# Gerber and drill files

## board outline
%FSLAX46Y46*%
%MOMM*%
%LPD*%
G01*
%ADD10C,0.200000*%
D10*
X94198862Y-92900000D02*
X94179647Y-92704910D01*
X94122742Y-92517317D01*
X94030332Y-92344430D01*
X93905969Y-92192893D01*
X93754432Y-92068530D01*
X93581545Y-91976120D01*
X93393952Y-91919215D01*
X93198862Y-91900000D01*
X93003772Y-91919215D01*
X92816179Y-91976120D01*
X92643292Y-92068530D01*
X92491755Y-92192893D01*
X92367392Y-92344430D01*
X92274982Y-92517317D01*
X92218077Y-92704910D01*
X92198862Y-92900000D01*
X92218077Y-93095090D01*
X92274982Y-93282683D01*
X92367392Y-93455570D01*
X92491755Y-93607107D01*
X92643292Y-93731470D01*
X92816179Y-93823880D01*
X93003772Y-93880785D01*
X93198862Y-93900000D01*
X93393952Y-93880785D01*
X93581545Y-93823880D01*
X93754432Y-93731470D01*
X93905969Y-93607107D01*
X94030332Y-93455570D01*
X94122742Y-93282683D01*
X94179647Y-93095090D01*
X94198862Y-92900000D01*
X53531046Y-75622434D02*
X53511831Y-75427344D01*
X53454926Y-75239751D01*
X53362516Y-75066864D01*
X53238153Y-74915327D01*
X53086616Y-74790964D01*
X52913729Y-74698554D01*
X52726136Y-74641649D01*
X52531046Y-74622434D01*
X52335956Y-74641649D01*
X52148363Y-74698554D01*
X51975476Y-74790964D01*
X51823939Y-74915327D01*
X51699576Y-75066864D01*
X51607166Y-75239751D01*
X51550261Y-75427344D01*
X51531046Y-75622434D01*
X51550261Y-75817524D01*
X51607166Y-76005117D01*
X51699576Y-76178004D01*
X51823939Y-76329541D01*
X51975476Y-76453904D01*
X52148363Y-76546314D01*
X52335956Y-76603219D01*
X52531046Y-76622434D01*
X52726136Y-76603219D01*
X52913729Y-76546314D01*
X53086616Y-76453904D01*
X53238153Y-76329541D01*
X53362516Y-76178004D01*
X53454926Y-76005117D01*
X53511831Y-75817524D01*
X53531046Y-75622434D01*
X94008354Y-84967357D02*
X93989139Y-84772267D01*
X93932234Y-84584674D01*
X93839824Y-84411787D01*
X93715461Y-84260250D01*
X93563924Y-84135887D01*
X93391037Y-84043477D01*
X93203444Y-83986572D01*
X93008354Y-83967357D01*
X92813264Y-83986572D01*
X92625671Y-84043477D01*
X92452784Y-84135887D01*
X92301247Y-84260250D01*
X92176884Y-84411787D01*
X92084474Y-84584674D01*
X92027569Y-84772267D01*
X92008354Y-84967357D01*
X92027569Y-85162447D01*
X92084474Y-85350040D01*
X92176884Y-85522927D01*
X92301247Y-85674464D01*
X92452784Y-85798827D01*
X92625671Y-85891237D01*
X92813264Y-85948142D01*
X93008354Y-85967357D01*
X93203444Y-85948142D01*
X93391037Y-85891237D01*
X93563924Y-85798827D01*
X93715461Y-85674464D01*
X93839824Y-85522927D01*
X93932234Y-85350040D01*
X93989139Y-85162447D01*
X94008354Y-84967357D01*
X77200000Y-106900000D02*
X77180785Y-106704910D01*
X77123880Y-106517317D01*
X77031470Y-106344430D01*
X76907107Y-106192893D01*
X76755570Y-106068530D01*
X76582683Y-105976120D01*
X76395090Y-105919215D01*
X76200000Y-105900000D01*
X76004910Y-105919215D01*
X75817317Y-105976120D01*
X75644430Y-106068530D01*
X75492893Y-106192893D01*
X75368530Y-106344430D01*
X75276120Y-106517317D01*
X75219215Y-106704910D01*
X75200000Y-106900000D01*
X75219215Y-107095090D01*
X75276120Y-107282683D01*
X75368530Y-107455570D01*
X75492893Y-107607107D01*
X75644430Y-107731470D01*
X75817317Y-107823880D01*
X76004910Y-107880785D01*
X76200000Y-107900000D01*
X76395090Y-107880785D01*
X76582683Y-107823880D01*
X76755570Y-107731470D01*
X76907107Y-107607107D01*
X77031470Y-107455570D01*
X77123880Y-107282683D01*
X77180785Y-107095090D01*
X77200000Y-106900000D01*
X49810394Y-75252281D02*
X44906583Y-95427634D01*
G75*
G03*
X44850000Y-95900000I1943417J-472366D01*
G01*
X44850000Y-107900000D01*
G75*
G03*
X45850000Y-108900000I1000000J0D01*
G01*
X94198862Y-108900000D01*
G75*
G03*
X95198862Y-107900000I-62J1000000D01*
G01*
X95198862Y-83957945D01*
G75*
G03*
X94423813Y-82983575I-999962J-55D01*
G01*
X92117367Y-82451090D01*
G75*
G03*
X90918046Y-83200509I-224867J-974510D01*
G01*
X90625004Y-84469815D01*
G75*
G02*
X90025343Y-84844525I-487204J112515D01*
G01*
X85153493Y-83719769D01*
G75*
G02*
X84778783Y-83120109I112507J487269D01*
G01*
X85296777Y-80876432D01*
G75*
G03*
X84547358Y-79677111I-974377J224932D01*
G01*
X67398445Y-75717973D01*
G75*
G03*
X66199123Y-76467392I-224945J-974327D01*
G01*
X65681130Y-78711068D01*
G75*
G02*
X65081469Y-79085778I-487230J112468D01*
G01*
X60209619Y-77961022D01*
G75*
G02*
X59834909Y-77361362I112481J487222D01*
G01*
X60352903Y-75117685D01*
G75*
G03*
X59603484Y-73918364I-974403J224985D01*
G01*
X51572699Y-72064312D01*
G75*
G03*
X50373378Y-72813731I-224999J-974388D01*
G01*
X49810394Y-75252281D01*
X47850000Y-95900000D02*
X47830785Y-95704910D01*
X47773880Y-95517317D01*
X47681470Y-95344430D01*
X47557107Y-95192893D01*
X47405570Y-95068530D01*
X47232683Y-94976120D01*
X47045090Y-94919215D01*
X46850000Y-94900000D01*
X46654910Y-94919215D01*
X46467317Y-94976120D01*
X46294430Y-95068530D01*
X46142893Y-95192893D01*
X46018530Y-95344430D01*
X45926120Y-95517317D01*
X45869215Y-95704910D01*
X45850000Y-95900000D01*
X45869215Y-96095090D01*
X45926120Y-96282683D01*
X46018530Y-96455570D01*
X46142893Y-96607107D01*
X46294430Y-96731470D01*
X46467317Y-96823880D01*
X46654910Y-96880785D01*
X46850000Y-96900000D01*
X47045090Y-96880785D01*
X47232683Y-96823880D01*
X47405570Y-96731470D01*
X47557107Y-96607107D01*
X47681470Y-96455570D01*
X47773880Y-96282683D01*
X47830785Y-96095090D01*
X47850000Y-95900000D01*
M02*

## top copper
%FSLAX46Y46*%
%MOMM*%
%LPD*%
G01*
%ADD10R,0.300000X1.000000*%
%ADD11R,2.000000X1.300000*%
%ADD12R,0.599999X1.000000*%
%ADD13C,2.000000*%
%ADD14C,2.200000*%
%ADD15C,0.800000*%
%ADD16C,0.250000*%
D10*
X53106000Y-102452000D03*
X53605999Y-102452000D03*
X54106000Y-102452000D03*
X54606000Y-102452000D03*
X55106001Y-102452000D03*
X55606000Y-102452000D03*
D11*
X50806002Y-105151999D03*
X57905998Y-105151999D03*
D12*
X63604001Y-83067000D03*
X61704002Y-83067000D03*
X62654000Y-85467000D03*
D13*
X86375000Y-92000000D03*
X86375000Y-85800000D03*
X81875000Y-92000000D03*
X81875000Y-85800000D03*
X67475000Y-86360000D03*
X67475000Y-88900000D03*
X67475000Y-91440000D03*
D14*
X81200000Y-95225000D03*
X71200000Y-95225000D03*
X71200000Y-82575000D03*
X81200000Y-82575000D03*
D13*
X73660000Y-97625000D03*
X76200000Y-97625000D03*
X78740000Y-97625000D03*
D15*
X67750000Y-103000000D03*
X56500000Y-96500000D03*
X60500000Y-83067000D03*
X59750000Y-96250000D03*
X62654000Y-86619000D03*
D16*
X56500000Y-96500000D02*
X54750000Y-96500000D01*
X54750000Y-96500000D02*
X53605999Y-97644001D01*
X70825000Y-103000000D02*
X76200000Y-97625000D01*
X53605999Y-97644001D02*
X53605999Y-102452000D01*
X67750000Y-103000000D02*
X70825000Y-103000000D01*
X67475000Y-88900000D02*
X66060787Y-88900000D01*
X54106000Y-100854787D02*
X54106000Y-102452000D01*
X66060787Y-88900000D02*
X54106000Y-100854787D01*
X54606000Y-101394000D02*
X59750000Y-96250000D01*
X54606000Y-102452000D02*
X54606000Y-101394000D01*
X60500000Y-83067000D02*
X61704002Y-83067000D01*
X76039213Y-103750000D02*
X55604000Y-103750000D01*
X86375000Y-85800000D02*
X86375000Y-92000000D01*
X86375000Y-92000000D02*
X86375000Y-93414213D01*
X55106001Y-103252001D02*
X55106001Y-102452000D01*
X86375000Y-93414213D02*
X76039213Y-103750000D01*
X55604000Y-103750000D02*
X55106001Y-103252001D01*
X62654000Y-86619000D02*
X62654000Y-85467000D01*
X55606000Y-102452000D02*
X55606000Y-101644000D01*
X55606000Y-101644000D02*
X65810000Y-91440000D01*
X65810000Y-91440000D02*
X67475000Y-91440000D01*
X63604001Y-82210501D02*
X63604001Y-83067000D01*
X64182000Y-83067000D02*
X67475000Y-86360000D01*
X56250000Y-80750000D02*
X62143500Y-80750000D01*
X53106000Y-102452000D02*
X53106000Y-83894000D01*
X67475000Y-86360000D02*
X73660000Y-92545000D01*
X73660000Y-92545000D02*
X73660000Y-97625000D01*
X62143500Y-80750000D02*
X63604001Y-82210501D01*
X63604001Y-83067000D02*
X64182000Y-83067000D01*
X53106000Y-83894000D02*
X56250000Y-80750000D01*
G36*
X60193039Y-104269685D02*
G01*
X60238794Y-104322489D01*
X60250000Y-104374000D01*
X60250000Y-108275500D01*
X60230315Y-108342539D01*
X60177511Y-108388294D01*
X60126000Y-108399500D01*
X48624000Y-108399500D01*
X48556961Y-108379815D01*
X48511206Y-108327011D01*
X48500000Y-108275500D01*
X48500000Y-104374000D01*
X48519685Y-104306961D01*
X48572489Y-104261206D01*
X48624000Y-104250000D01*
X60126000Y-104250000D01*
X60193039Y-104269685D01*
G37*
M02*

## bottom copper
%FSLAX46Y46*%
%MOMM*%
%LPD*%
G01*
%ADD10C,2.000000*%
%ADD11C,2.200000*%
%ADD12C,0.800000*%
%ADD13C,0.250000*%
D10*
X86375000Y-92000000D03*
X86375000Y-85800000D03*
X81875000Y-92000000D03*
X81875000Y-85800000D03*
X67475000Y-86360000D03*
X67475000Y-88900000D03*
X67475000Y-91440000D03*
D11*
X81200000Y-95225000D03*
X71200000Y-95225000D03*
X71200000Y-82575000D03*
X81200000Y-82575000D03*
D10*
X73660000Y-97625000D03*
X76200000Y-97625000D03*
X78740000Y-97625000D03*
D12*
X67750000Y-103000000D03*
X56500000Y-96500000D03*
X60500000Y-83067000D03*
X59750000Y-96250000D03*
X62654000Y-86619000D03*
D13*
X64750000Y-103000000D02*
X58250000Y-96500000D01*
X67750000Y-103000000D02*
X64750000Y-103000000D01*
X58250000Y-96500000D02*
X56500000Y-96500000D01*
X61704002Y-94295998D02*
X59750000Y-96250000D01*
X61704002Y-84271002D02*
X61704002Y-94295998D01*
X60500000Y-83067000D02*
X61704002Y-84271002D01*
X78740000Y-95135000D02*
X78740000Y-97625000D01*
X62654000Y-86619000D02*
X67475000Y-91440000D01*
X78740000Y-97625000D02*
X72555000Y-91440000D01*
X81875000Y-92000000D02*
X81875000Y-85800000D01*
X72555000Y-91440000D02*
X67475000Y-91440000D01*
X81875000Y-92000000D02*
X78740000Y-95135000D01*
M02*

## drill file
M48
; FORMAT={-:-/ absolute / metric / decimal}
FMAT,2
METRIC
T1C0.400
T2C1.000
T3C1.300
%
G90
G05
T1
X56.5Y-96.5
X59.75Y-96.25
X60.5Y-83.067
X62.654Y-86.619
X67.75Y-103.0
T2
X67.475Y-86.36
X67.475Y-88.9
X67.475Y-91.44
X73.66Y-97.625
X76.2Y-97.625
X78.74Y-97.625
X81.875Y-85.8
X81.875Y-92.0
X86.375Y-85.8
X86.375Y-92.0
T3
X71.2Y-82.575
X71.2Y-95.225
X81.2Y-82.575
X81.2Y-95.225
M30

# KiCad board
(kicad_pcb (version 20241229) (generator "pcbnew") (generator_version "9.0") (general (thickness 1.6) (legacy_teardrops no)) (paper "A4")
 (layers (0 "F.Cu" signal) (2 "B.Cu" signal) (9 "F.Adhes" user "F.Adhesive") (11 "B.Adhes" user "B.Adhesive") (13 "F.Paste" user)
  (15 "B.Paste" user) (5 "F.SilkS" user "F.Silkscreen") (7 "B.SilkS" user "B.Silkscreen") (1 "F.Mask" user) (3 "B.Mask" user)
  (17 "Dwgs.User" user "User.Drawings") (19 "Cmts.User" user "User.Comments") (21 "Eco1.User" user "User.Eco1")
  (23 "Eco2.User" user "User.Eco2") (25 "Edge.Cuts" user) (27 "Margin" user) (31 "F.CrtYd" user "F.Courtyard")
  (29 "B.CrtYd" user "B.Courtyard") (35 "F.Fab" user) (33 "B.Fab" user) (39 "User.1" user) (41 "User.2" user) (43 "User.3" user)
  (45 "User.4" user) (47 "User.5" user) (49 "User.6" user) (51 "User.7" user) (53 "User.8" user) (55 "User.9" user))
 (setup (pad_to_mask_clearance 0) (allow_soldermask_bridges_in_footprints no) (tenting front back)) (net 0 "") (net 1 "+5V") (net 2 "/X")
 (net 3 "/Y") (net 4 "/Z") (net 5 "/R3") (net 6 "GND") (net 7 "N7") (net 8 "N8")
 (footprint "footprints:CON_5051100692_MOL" (layer "F.Cu") (at 54.356 104.902)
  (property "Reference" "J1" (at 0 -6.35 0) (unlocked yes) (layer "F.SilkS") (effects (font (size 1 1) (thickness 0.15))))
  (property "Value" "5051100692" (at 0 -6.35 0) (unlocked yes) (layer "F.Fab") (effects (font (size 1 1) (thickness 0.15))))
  (pad "1" smd rect (at -1.25 -2.45) (size 0.3 1) (layers "F.Cu" "F.Mask" "F.Paste") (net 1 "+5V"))
  (pad "2" smd rect (at -0.750001 -2.45) (size 0.3 1) (layers "F.Cu" "F.Mask" "F.Paste") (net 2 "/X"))
  (pad "3" smd rect (at -0.25 -2.45) (size 0.3 1) (layers "F.Cu" "F.Mask" "F.Paste") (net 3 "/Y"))
  (pad "4" smd rect (at 0.25 -2.45) (size 0.3 1) (layers "F.Cu" "F.Mask" "F.Paste") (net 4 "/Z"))
  (pad "5" smd rect (at 0.750001 -2.45) (size 0.3 1) (layers "F.Cu" "F.Mask" "F.Paste") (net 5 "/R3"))
  (pad "6" smd rect (at 1.25 -2.45) (size 0.3 1) (layers "F.Cu" "F.Mask" "F.Paste") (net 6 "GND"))
  (pad "P1" smd rect (at -3.549998 0.249999) (size 2 1.3) (layers "F.Cu" "F.Mask" "F.Paste") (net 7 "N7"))
  (pad "P2" smd rect (at 3.549998 0.249999) (size 2 1.3) (layers "F.Cu" "F.Mask" "F.Paste") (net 7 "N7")))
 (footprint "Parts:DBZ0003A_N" (layer "F.Cu") (at 62.654 84.267 -90)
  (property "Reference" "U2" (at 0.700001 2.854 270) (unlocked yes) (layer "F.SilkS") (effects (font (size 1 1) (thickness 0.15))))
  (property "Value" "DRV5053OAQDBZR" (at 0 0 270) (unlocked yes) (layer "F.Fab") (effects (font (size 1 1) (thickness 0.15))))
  (pad "1" smd rect (at -1.2 -0.950001) (size 0.599999 1) (layers "F.Cu" "F.Mask" "F.Paste") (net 1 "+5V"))
  (pad "2" smd rect (at -1.2 0.949998) (size 0.599999 1) (layers "F.Cu" "F.Mask" "F.Paste") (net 4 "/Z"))
  (pad "3" smd rect (at 1.2 0) (size 0.599999 1) (layers "F.Cu" "F.Mask" "F.Paste") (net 6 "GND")))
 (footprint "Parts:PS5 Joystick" (layer "B.Cu") (at 76.2 88.9 180)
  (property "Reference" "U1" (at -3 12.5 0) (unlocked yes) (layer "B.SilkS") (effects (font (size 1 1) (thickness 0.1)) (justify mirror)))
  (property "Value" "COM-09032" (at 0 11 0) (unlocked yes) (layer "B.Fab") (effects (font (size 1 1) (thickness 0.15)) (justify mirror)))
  (pad "B1A" thru_hole circle (at -10.175 -3.1 180) (size 2 2) (drill 1) (layers "*.Cu" "*.Mask") (remove_unused_layers no) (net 5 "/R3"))
  (pad "B1A" thru_hole circle (at -10.175 3.1 180) (size 2 2) (drill 1) (layers "*.Cu" "*.Mask") (remove_unused_layers no) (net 5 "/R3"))
  (pad "B2A" thru_hole circle (at -5.675 -3.1 180) (size 2 2) (drill 1) (layers "*.Cu" "*.Mask") (remove_unused_layers no) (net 6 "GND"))
  (pad "B2A" thru_hole circle (at -5.675 3.1 180) (size 2 2) (drill 1) (layers "*.Cu" "*.Mask") (remove_unused_layers no) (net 6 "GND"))
  (pad "H1" thru_hole circle (at 8.725 2.54 180) (size 2 2) (drill 1) (layers "*.Cu" "*.Mask") (remove_unused_layers no) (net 1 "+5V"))
  (pad "H2" thru_hole circle (at 8.725 0 180) (size 2 2) (drill 1) (layers "*.Cu" "*.Mask") (remove_unused_layers no) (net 3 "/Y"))
  (pad "H3" thru_hole circle (at 8.725 -2.54 180) (size 2 2) (drill 1) (layers "*.Cu" "*.Mask") (remove_unused_layers no) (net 6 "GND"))
  (pad "S1" thru_hole circle (at -5 -6.325 180) (size 2.2 2.2) (drill 1.3) (layers "*.Cu" "*.Mask") (remove_unused_layers no) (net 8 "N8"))
  (pad "S2" thru_hole circle (at 5 -6.325 180) (size 2.2 2.2) (drill 1.3) (layers "*.Cu" "*.Mask") (remove_unused_layers no) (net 8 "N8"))
  (pad "S3" thru_hole circle (at 5 6.325 180) (size 2.2 2.2) (drill 1.3) (layers "*.Cu" "*.Mask") (remove_unused_layers no) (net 8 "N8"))
  (pad "S4" thru_hole circle (at -5 6.325 180) (size 2.2 2.2) (drill 1.3) (layers "*.Cu" "*.Mask") (remove_unused_layers no) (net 8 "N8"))
  (pad "V1" thru_hole circle (at 2.54 -8.725 180) (size 2 2) (drill 1) (layers "*.Cu" "*.Mask") (remove_unused_layers no) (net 1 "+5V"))
  (pad "V2" thru_hole circle (at 0 -8.725 180) (size 2 2) (drill 1) (layers "*.Cu" "*.Mask") (remove_unused_layers no) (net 2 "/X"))
  (pad "V3" thru_hole circle (at -2.54 -8.725 180) (size 2 2) (drill 1) (layers "*.Cu" "*.Mask") (remove_unused_layers no) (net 6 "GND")))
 (gr_poly
  (pts (xy 94.198862 92.9) (xy 94.179647 92.70491) (xy 94.122742 92.517317) (xy 94.030332 92.34443) (xy 93.905969 92.192893)
   (xy 93.754432 92.06853) (xy 93.581545 91.97612) (xy 93.393952 91.919215) (xy 93.198862 91.9) (xy 93.003772 91.919215)
   (xy 92.816179 91.97612) (xy 92.643292 92.06853) (xy 92.491755 92.192893) (xy 92.367392 92.34443) (xy 92.274982 92.517317)
   (xy 92.218077 92.70491) (xy 92.198862 92.9) (xy 92.218077 93.09509) (xy 92.274982 93.282683) (xy 92.367392 93.45557)
   (xy 92.491755 93.607107) (xy 92.643292 93.73147) (xy 92.816179 93.82388) (xy 93.003772 93.880785) (xy 93.198862 93.9)
   (xy 93.393952 93.880785) (xy 93.581545 93.82388) (xy 93.754432 93.73147) (xy 93.905969 93.607107) (xy 94.030332 93.45557)
   (xy 94.122742 93.282683) (xy 94.179647 93.09509) (xy 94.198862 92.9))
  (stroke (width 0.2) (type solid)) (fill no) (layer "Edge.Cuts"))
 (gr_poly
  (pts (xy 53.531046 75.622434) (xy 53.511831 75.427344) (xy 53.454926 75.239751) (xy 53.362516 75.066864) (xy 53.238153 74.915327)
   (xy 53.086616 74.790964) (xy 52.913729 74.698554) (xy 52.726136 74.641649) (xy 52.531046 74.622434) (xy 52.335956 74.641649)
   (xy 52.148363 74.698554) (xy 51.975476 74.790964) (xy 51.823939 74.915327) (xy 51.699576 75.066864) (xy 51.607166 75.239751)
   (xy 51.550261 75.427344) (xy 51.531046 75.622434) (xy 51.550261 75.817524) (xy 51.607166 76.005117) (xy 51.699576 76.178004)
   (xy 51.823939 76.329541) (xy 51.975476 76.453904) (xy 52.148363 76.546314) (xy 52.335956 76.603219) (xy 52.531046 76.622434)
   (xy 52.726136 76.603219) (xy 52.913729 76.546314) (xy 53.086616 76.453904) (xy 53.238153 76.329541) (xy 53.362516 76.178004)
   (xy 53.454926 76.005117) (xy 53.511831 75.817524) (xy 53.531046 75.622434))
  (stroke (width 0.2) (type solid)) (fill no) (layer "Edge.Cuts"))
 (gr_poly
  (pts (xy 94.008354 84.967357) (xy 93.989139 84.772267) (xy 93.932234 84.584674) (xy 93.839824 84.411787) (xy 93.715461 84.26025)
   (xy 93.563924 84.135887) (xy 93.391037 84.043477) (xy 93.203444 83.986572) (xy 93.008354 83.967357) (xy 92.813264 83.986572)
   (xy 92.625671 84.043477) (xy 92.452784 84.135887) (xy 92.301247 84.26025) (xy 92.176884 84.411787) (xy 92.084474 84.584674)
   (xy 92.027569 84.772267) (xy 92.008354 84.967357) (xy 92.027569 85.162447) (xy 92.084474 85.35004) (xy 92.176884 85.522927)
   (xy 92.301247 85.674464) (xy 92.452784 85.798827) (xy 92.625671 85.891237) (xy 92.813264 85.948142) (xy 93.008354 85.967357)
   (xy 93.203444 85.948142) (xy 93.391037 85.891237) (xy 93.563924 85.798827) (xy 93.715461 85.674464) (xy 93.839824 85.522927)
   (xy 93.932234 85.35004) (xy 93.989139 85.162447) (xy 94.008354 84.967357))
  (stroke (width 0.2) (type solid)) (fill no) (layer "Edge.Cuts"))
 (gr_poly
  (pts (xy 77.2 106.9) (xy 77.180785 106.70491) (xy 77.12388 106.517317) (xy 77.03147 106.34443) (xy 76.907107 106.192893)
   (xy 76.75557 106.06853) (xy 76.582683 105.97612) (xy 76.39509 105.919215) (xy 76.2 105.9) (xy 76.00491 105.919215)
   (xy 75.817317 105.97612) (xy 75.64443 106.06853) (xy 75.492893 106.192893) (xy 75.36853 106.34443) (xy 75.27612 106.517317)
   (xy 75.219215 106.70491) (xy 75.2 106.9) (xy 75.219215 107.09509) (xy 75.27612 107.282683) (xy 75.36853 107.45557)
   (xy 75.492893 107.607107) (xy 75.64443 107.73147) (xy 75.817317 107.82388) (xy 76.00491 107.880785) (xy 76.2 107.9)
   (xy 76.39509 107.880785) (xy 76.582683 107.82388) (xy 76.75557 107.73147) (xy 76.907107 107.607107) (xy 77.03147 107.45557)
   (xy 77.12388 107.282683) (xy 77.180785 107.09509) (xy 77.2 106.9))
  (stroke (width 0.2) (type solid)) (fill no) (layer "Edge.Cuts"))
 (gr_poly
  (pts (xy 49.810394 75.252281)
   (arc (start 44.906583 95.427634) (mid 44.864196 95.662129) (end 44.85 95.9))
   (arc (start 44.85 107.9) (mid 45.142893 108.607107) (end 45.85 108.9))
   (arc (start 94.198862 108.9) (mid 94.905966 108.607093) (end 95.198862 107.9))
   (arc (start 95.198862 83.957945) (mid 94.981467 83.335431) (end 94.423813 82.983575))
   (arc (start 92.117367 82.45109) (mid 91.362505 82.577445) (end 90.918046 83.200509))
   (arc (start 90.625004 84.469815) (mid 90.402771 84.781349) (end 90.025343 84.844525))
   (arc (start 85.153493 83.719769) (mid 84.841972 83.497537) (end 84.778783 83.120109))
   (arc (start 85.296777 80.876432) (mid 85.170456 80.121561) (end 84.547358 79.677111))
   (arc (start 67.398445 75.717973) (mid 66.643574 75.844295) (end 66.199123 76.467392))
   (arc (start 65.68113 78.711068) (mid 65.458904 79.022617) (end 65.081469 79.085778))
   (arc (start 60.209619 77.961022) (mid 59.89807 77.738797) (end 59.834909 77.361362))
   (arc (start 60.352903 75.117685) (mid 60.226581 74.362815) (end 59.603484 73.918364))
   (arc (start 51.572699 72.064312) (mid 50.817829 72.190634) (end 50.373378 72.813731)))
  (stroke (width 0.2) (type solid)) (fill no) (layer "Edge.Cuts"))
 (gr_poly
  (pts (xy 47.85 95.9) (xy 47.830785 95.70491) (xy 47.77388 95.517317) (xy 47.68147 95.34443) (xy 47.557107 95.192893)
   (xy 47.40557 95.06853) (xy 47.232683 94.97612) (xy 47.04509 94.919215) (xy 46.85 94.9) (xy 46.65491 94.919215) (xy 46.467317 94.97612)
   (xy 46.29443 95.06853) (xy 46.142893 95.192893) (xy 46.01853 95.34443) (xy 45.92612 95.517317) (xy 45.869215 95.70491) (xy 45.85 95.9)
   (xy 45.869215 96.09509) (xy 45.92612 96.282683) (xy 46.01853 96.45557) (xy 46.142893 96.607107) (xy 46.29443 96.73147)
   (xy 46.467317 96.82388) (xy 46.65491 96.880785) (xy 46.85 96.9) (xy 47.04509 96.880785) (xy 47.232683 96.82388) (xy 47.40557 96.73147)
   (xy 47.557107 96.607107) (xy 47.68147 96.45557) (xy 47.77388 96.282683) (xy 47.830785 96.09509) (xy 47.85 95.9))
  (stroke (width 0.2) (type solid)) (fill no) (layer "Edge.Cuts"))
 (segment (start 56.5 96.5) (end 54.75 96.5) (width 0.25) (layer "F.Cu") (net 2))
 (segment (start 54.75 96.5) (end 53.605999 97.644001) (width 0.25) (layer "F.Cu") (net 2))
 (segment (start 70.825 103) (end 76.2 97.625) (width 0.25) (layer "F.Cu") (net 2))
 (segment (start 53.605999 97.644001) (end 53.605999 102.452) (width 0.25) (layer "F.Cu") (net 2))
 (segment (start 67.75 103) (end 70.825 103) (width 0.25) (layer "F.Cu") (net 2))
 (via (at 67.75 103) (size 0.8) (drill 0.4) (layers "F.Cu" "B.Cu") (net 2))
 (via (at 56.5 96.5) (size 0.8) (drill 0.4) (layers "F.Cu" "B.Cu") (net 2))
 (segment (start 64.75 103) (end 58.25 96.5) (width 0.25) (layer "B.Cu") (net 2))
 (segment (start 67.75 103) (end 64.75 103) (width 0.25) (layer "B.Cu") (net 2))
 (segment (start 58.25 96.5) (end 56.5 96.5) (width 0.25) (layer "B.Cu") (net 2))
 (segment (start 67.475 88.9) (end 66.060787 88.9) (width 0.25) (layer "F.Cu") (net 3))
 (segment (start 54.106 100.854787) (end 54.106 102.452) (width 0.25) (layer "F.Cu") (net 3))
 (segment (start 66.060787 88.9) (end 54.106 100.854787) (width 0.25) (layer "F.Cu") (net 3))
 (segment (start 54.606 101.394) (end 59.75 96.25) (width 0.25) (layer "F.Cu") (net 4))
 (segment (start 54.606 102.452) (end 54.606 101.394) (width 0.25) (layer "F.Cu") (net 4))
 (segment (start 60.5 83.067) (end 61.704002 83.067) (width 0.25) (layer "F.Cu") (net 4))
 (via (at 60.5 83.067) (size 0.8) (drill 0.4) (layers "F.Cu" "B.Cu") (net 4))
 (via (at 59.75 96.25) (size 0.8) (drill 0.4) (layers "F.Cu" "B.Cu") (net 4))
 (segment (start 61.704002 94.295998) (end 59.75 96.25) (width 0.25) (layer "B.Cu") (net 4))
 (segment (start 61.704002 84.271002) (end 61.704002 94.295998) (width 0.25) (layer "B.Cu") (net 4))
 (segment (start 60.5 83.067) (end 61.704002 84.271002) (width 0.25) (layer "B.Cu") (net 4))
 (segment (start 76.039213 103.75) (end 55.604 103.75) (width 0.25) (layer "F.Cu") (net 5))
 (segment (start 86.375 85.8) (end 86.375 92) (width 0.25) (layer "F.Cu") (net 5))
 (segment (start 86.375 92) (end 86.375 93.414213) (width 0.25) (layer "F.Cu") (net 5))
 (segment (start 55.106001 103.252001) (end 55.106001 102.452) (width 0.25) (layer "F.Cu") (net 5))
 (segment (start 86.375 93.414213) (end 76.039213 103.75) (width 0.25) (layer "F.Cu") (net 5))
 (segment (start 55.604 103.75) (end 55.106001 103.252001) (width 0.25) (layer "F.Cu") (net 5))
 (segment (start 62.654 86.619) (end 62.654 85.467) (width 0.25) (layer "F.Cu") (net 6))
 (segment (start 55.606 102.452) (end 55.606 101.644) (width 0.25) (layer "F.Cu") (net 6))
 (segment (start 55.606 101.644) (end 65.81 91.44) (width 0.25) (layer "F.Cu") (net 6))
 (segment (start 65.81 91.44) (end 67.475 91.44) (width 0.25) (layer "F.Cu") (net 6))
 (via (at 62.654 86.619) (size 0.8) (drill 0.4) (layers "F.Cu" "B.Cu") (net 6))
 (segment (start 78.74 95.135) (end 78.74 97.625) (width 0.25) (layer "B.Cu") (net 6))
 (segment (start 62.654 86.619) (end 67.475 91.44) (width 0.25) (layer "B.Cu") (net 6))
 (segment (start 78.74 97.625) (end 72.555 91.44) (width 0.25) (layer "B.Cu") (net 6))
 (segment (start 81.875 92) (end 81.875 85.8) (width 0.25) (layer "B.Cu") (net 6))
 (segment (start 72.555 91.44) (end 67.475 91.44) (width 0.25) (layer "B.Cu") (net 6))
 (segment (start 81.875 92) (end 78.74 95.135) (width 0.25) (layer "B.Cu") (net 6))
 (segment (start 63.604001 82.210501) (end 63.604001 83.067) (width 0.25) (layer "F.Cu") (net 1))
 (segment (start 64.182 83.067) (end 67.475 86.36) (width 0.25) (layer "F.Cu") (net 1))
 (segment (start 56.25 80.75) (end 62.1435 80.75) (width 0.25) (layer "F.Cu") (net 1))
 (segment (start 53.106 102.452) (end 53.106 83.894) (width 0.25) (layer "F.Cu") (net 1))
 (segment (start 67.475 86.36) (end 73.66 92.545) (width 0.25) (layer "F.Cu") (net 1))
 (segment (start 73.66 92.545) (end 73.66 97.625) (width 0.25) (layer "F.Cu") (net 1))
 (segment (start 62.1435 80.75) (end 63.604001 82.210501) (width 0.25) (layer "F.Cu") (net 1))
 (segment (start 63.604001 83.067) (end 64.182 83.067) (width 0.25) (layer "F.Cu") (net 1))
 (segment (start 53.106 83.894) (end 56.25 80.75) (width 0.25) (layer "F.Cu") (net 1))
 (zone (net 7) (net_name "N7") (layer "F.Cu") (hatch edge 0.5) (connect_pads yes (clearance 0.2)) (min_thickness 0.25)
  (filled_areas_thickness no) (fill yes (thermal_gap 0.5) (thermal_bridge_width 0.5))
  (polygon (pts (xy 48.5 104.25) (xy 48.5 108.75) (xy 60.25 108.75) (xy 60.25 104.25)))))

